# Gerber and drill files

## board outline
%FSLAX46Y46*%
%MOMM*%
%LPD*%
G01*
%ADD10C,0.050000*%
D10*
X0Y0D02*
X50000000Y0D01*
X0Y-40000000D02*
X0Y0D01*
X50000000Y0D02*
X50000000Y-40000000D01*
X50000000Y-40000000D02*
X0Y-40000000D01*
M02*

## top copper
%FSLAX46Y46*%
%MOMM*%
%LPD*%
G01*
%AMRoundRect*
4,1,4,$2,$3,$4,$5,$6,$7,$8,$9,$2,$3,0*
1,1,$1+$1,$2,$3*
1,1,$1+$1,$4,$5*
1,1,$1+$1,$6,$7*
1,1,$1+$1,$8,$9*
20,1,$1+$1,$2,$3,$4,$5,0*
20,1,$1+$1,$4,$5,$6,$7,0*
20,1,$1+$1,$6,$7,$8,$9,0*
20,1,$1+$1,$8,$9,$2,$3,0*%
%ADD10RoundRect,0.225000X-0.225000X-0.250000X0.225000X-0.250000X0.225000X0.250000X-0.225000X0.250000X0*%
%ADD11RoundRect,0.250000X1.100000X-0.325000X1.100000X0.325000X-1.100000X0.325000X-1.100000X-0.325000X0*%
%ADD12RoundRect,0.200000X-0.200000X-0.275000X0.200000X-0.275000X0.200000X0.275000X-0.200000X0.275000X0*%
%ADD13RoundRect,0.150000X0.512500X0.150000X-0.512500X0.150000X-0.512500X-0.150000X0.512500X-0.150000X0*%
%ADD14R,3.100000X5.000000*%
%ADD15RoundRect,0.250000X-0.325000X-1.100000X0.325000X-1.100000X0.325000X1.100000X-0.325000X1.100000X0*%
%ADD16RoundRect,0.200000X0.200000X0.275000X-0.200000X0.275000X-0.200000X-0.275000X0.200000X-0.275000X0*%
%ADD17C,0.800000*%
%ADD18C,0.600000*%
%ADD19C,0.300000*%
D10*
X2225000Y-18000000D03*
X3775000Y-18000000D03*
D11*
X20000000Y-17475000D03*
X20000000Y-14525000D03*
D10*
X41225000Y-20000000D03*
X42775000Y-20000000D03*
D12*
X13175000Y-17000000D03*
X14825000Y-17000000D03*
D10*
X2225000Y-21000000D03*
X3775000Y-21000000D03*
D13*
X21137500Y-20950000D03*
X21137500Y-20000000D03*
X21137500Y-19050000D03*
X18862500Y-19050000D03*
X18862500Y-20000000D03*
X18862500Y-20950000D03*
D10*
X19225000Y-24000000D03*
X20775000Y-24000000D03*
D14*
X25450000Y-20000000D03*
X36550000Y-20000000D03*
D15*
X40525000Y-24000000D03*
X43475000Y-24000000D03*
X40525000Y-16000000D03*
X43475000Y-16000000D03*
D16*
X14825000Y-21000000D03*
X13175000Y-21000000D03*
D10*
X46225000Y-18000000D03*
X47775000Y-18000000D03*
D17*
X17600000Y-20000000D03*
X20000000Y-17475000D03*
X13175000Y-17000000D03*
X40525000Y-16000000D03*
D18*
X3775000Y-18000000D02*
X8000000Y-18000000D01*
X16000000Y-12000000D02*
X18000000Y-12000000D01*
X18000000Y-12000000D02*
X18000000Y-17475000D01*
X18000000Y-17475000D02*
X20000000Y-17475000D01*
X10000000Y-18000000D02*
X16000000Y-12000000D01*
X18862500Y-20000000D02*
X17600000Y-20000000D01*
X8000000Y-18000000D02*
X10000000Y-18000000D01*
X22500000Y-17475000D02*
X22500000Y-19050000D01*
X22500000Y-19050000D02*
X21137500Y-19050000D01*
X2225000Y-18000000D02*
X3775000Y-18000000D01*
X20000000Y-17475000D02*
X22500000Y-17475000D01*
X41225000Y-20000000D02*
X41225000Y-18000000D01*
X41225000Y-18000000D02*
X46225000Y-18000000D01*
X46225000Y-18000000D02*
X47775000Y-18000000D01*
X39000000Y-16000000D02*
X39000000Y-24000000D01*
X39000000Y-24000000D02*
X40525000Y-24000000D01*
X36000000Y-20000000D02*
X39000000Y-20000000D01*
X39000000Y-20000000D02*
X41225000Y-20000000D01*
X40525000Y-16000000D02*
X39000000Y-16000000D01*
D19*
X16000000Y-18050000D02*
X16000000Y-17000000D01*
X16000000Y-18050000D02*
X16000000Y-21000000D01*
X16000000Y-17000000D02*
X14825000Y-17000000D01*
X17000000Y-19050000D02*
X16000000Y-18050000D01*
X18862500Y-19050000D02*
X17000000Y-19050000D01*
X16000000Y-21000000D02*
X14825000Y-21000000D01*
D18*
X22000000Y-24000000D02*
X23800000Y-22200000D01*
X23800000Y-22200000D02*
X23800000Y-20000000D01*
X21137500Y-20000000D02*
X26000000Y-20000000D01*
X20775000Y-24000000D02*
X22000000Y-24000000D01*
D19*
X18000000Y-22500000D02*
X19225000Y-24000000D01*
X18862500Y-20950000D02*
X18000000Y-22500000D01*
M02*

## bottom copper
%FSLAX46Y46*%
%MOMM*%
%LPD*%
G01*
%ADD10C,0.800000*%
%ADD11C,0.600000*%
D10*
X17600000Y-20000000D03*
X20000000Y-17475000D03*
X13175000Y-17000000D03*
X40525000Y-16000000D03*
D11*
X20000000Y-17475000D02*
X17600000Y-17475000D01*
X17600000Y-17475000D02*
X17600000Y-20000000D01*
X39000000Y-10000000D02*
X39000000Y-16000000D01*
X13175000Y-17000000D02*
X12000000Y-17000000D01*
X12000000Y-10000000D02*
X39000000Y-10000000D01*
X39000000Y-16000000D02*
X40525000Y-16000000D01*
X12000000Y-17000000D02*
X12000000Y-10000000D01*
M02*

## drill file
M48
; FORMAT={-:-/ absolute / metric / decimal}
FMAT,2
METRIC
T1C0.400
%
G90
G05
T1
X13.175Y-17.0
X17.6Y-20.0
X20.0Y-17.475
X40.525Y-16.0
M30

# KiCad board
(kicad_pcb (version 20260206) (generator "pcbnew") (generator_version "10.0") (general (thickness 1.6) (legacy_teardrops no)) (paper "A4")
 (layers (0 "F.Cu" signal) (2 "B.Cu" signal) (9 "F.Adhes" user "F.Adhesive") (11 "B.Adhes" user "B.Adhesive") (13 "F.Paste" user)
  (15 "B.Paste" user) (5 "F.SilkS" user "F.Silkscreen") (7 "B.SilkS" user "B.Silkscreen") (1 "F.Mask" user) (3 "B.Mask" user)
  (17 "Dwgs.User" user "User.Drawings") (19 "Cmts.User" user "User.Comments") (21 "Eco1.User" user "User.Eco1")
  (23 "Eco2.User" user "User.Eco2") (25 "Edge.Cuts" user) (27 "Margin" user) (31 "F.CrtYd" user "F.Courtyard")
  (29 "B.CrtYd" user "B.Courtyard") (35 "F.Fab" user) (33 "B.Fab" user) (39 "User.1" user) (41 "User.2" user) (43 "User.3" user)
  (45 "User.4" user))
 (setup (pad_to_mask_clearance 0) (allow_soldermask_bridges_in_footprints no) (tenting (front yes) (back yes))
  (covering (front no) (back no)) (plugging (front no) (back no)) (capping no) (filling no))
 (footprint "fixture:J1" (layer "F.Cu") (at 3 18)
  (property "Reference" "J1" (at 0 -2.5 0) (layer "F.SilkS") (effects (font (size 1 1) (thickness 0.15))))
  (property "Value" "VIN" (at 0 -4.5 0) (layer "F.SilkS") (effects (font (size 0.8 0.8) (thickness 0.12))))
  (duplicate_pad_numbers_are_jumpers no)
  (pad "1" smd roundrect (at -0.775 0) (size 0.9 0.95) (layers "F.Cu" "F.Mask" "F.Paste") (roundrect_rratio 0.25) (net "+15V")
   (thermal_bridge_angle 45))
  (pad "2" smd roundrect (at 0.775 0) (size 0.9 0.95) (layers "F.Cu" "F.Mask" "F.Paste") (roundrect_rratio 0.25) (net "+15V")
   (thermal_bridge_angle 45)))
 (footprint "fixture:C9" (layer "F.Cu") (at 20 16 90)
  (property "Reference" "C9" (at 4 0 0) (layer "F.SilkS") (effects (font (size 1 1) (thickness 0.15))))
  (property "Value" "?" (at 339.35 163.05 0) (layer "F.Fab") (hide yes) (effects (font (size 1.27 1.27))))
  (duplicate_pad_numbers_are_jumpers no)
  (pad "1" smd roundrect (at -1.475 0 90) (size 1.15 2.7) (layers "F.Cu" "F.Mask" "F.Paste") (roundrect_rratio 0.217391) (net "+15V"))
  (pad "2" smd roundrect (at 1.475 0 90) (size 1.15 2.7) (layers "F.Cu" "F.Mask" "F.Paste") (roundrect_rratio 0.217391) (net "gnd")))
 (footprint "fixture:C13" (layer "F.Cu") (at 42 20)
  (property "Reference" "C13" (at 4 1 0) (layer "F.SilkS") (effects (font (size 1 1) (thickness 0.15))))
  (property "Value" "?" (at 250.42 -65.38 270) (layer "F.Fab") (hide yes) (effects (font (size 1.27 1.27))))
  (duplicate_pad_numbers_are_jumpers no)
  (pad "1" smd roundrect (at -0.775 0) (size 0.9 0.95) (layers "F.Cu" "F.Mask" "F.Paste") (roundrect_rratio 0.25) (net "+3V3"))
  (pad "2" smd roundrect (at 0.775 0) (size 0.9 0.95) (layers "F.Cu" "F.Mask" "F.Paste") (roundrect_rratio 0.25) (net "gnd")))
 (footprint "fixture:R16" (layer "F.Cu") (at 14 17)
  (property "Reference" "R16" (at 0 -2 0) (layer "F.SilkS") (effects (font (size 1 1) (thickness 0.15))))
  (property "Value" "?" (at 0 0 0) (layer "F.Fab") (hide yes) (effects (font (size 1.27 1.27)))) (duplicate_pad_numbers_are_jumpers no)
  (pad "1" smd roundrect (at -0.825 0) (size 0.8 0.95) (layers "F.Cu" "F.Mask" "F.Paste") (roundrect_rratio 0.25) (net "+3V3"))
  (pad "2" smd roundrect (at 0.825 0) (size 0.8 0.95) (layers "F.Cu" "F.Mask" "F.Paste") (roundrect_rratio 0.25) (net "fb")))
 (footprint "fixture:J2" (layer "F.Cu") (at 3 21)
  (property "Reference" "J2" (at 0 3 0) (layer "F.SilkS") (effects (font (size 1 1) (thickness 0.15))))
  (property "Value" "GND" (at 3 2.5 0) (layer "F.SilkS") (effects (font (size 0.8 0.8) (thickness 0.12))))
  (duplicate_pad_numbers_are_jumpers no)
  (pad "1" smd roundrect (at -0.775 0) (size 0.9 0.95) (layers "F.Cu" "F.Mask" "F.Paste") (roundrect_rratio 0.25) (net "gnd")
   (thermal_bridge_angle 45))
  (pad "2" smd roundrect (at 0.775 0) (size 0.9 0.95) (layers "F.Cu" "F.Mask" "F.Paste") (roundrect_rratio 0.25) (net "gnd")
   (thermal_bridge_angle 45)))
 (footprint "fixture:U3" (layer "F.Cu") (at 20 20 180)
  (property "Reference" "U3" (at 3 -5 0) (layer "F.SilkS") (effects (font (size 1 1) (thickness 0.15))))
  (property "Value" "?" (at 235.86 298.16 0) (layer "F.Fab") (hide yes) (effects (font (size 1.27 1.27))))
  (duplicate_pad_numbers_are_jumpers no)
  (pad "1" smd roundrect (at -1.1375 -0.95 180) (size 1.325 0.6) (layers "F.Cu" "F.Mask" "F.Paste") (roundrect_rratio 0.25) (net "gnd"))
  (pad "2" smd roundrect (at -1.1375 0 180) (size 1.325 0.6) (layers "F.Cu" "F.Mask" "F.Paste") (roundrect_rratio 0.25) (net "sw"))
  (pad "3" smd roundrect (at -1.1375 0.95 180) (size 1.325 0.6) (layers "F.Cu" "F.Mask" "F.Paste") (roundrect_rratio 0.25) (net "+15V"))
  (pad "4" smd roundrect (at 1.1375 0.95 180) (size 1.325 0.6) (layers "F.Cu" "F.Mask" "F.Paste") (roundrect_rratio 0.25) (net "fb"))
  (pad "5" smd roundrect (at 1.1375 0 180) (size 1.325 0.6) (layers "F.Cu" "F.Mask" "F.Paste") (roundrect_rratio 0.25) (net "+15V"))
  (pad "6" smd roundrect (at 1.1375 -0.95 180) (size 1.325 0.6) (layers "F.Cu" "F.Mask" "F.Paste") (roundrect_rratio 0.25) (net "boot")))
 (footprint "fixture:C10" (layer "F.Cu") (at 20 24)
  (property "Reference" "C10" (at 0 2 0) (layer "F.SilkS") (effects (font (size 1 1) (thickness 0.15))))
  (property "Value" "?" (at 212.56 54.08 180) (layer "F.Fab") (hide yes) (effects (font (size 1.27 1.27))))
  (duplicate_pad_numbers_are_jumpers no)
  (pad "1" smd roundrect (at -0.775 0) (size 0.9 0.95) (layers "F.Cu" "F.Mask" "F.Paste") (roundrect_rratio 0.25) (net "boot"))
  (pad "2" smd roundrect (at 0.775 0) (size 0.9 0.95) (layers "F.Cu" "F.Mask" "F.Paste") (roundrect_rratio 0.25) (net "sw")))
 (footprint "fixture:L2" (layer "F.Cu") (at 31 20)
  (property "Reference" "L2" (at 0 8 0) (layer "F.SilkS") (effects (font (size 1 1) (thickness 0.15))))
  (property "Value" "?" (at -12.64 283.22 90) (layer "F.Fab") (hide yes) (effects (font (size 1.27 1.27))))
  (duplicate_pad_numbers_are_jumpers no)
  (pad "1" smd rect (at -5.55 0) (size 3.1 5) (layers "F.Cu" "F.Mask" "F.Paste") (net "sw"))
  (pad "2" smd rect (at 5.55 0) (size 3.1 5) (layers "F.Cu" "F.Mask" "F.Paste") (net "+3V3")))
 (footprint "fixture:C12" (layer "F.Cu") (at 42 24)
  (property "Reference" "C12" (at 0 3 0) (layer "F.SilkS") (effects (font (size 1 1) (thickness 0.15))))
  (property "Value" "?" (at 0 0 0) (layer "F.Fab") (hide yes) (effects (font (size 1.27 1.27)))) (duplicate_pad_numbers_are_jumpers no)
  (pad "1" smd roundrect (at -1.475 0) (size 1.15 2.7) (layers "F.Cu" "F.Mask" "F.Paste") (roundrect_rratio 0.217391) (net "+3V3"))
  (pad "2" smd roundrect (at 1.475 0) (size 1.15 2.7) (layers "F.Cu" "F.Mask" "F.Paste") (roundrect_rratio 0.217391) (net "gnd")))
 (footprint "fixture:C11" (layer "F.Cu") (at 42 16)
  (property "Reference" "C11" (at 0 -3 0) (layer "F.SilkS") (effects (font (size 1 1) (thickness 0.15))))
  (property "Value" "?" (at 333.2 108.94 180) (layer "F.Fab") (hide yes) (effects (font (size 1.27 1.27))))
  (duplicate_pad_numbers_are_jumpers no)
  (pad "1" smd roundrect (at -1.475 0) (size 1.15 2.7) (layers "F.Cu" "F.Mask" "F.Paste") (roundrect_rratio 0.217391) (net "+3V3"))
  (pad "2" smd roundrect (at 1.475 0) (size 1.15 2.7) (layers "F.Cu" "F.Mask" "F.Paste") (roundrect_rratio 0.217391) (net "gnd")))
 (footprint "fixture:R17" (layer "F.Cu") (at 14 21 180)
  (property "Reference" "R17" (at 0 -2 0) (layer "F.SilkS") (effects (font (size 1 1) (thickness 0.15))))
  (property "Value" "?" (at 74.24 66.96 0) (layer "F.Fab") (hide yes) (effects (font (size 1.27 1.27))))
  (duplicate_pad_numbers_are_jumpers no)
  (pad "1" smd roundrect (at -0.825 0 180) (size 0.8 0.95) (layers "F.Cu" "F.Mask" "F.Paste") (roundrect_rratio 0.25) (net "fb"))
  (pad "2" smd roundrect (at 0.825 0 180) (size 0.8 0.95) (layers "F.Cu" "F.Mask" "F.Paste") (roundrect_rratio 0.25) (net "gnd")))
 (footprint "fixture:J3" (layer "F.Cu") (at 47 18)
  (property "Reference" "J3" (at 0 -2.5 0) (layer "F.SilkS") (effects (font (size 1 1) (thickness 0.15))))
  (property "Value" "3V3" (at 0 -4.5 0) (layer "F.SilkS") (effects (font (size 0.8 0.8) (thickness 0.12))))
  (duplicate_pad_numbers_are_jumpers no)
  (pad "1" smd roundrect (at -0.775 0) (size 0.9 0.95) (layers "F.Cu" "F.Mask" "F.Paste") (roundrect_rratio 0.25) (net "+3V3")
   (thermal_bridge_angle 45))
  (pad "2" smd roundrect (at 0.775 0) (size 0.9 0.95) (layers "F.Cu" "F.Mask" "F.Paste") (roundrect_rratio 0.25) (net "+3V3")
   (thermal_bridge_angle 45)))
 (gr_line (start 0 0) (end 50 0) (stroke (width 0.05) (type default)) (layer "Edge.Cuts"))
 (gr_line (start 0 40) (end 0 0) (stroke (width 0.05) (type default)) (layer "Edge.Cuts"))
 (gr_line (start 50 0) (end 50 40) (stroke (width 0.05) (type default)) (layer "Edge.Cuts"))
 (gr_line (start 50 40) (end 0 40) (stroke (width 0.05) (type default)) (layer "Edge.Cuts"))
 (segment (start 3.775 18) (end 8 18) (width 0.6) (layer "F.Cu") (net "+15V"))
 (segment (start 16 12) (end 18 12) (width 0.6) (layer "F.Cu") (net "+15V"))
 (segment (start 18 12) (end 18 17.475) (width 0.6) (layer "F.Cu") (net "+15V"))
 (segment (start 18 17.475) (end 20 17.475) (width 0.6) (layer "F.Cu") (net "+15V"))
 (segment (start 10 18) (end 16 12) (width 0.6) (layer "F.Cu") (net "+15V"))
 (segment (start 18.8625 20) (end 17.6 20) (width 0.6) (layer "F.Cu") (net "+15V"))
 (segment (start 8 18) (end 10 18) (width 0.6) (layer "F.Cu") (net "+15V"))
 (segment (start 22.5 17.475) (end 22.5 19.05) (width 0.6) (layer "F.Cu") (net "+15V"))
 (segment (start 22.5 19.05) (end 21.1375 19.05) (width 0.6) (layer "F.Cu") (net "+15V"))
 (segment (start 2.225 18) (end 3.775 18) (width 0.6) (layer "F.Cu") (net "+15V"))
 (segment (start 20 17.475) (end 22.5 17.475) (width 0.6) (layer "F.Cu") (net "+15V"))
 (via (at 17.6 20) (size 0.8) (drill 0.4) (layers "F.Cu" "B.Cu") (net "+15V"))
 (via (at 20 17.475) (size 0.8) (drill 0.4) (layers "F.Cu" "B.Cu") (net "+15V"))
 (segment (start 20 17.475) (end 17.6 17.475) (width 0.6) (layer "B.Cu") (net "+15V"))
 (segment (start 17.6 17.475) (end 17.6 20) (width 0.6) (layer "B.Cu") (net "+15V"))
 (segment (start 41.225 20) (end 41.225 18) (width 0.6) (layer "F.Cu") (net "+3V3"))
 (segment (start 41.225 18) (end 46.225 18) (width 0.6) (layer "F.Cu") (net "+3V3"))
 (segment (start 46.225 18) (end 47.775 18) (width 0.6) (layer "F.Cu") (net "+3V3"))
 (segment (start 39 16) (end 39 24) (width 0.6) (layer "F.Cu") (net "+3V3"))
 (segment (start 39 24) (end 40.525 24) (width 0.6) (layer "F.Cu") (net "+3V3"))
 (segment (start 36 20) (end 39 20) (width 0.6) (layer "F.Cu") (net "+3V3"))
 (segment (start 39 20) (end 41.225 20) (width 0.6) (layer "F.Cu") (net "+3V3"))
 (segment (start 40.525 16) (end 39 16) (width 0.6) (layer "F.Cu") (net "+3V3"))
 (via (at 13.175 17) (size 0.8) (drill 0.4) (layers "F.Cu" "B.Cu") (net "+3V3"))
 (via (at 40.525 16) (size 0.8) (drill 0.4) (layers "F.Cu" "B.Cu") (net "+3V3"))
 (segment (start 39 10) (end 39 16) (width 0.6) (layer "B.Cu") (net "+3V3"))
 (segment (start 13.175 17) (end 12 17) (width 0.6) (layer "B.Cu") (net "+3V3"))
 (segment (start 12 10) (end 39 10) (width 0.6) (layer "B.Cu") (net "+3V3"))
 (segment (start 39 16) (end 40.525 16) (width 0.6) (layer "B.Cu") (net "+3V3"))
 (segment (start 12 17) (end 12 10) (width 0.6) (layer "B.Cu") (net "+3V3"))
 (segment (start 16 18.05) (end 16 17) (width 0.3) (layer "F.Cu") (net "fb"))
 (segment (start 16 18.05) (end 16 21) (width 0.3) (layer "F.Cu") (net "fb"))
 (segment (start 16 17) (end 14.825 17) (width 0.3) (layer "F.Cu") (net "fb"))
 (segment (start 17 19.05) (end 16 18.05) (width 0.3) (layer "F.Cu") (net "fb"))
 (segment (start 18.8625 19.05) (end 17 19.05) (width 0.3) (layer "F.Cu") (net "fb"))
 (segment (start 16 21) (end 14.825 21) (width 0.3) (layer "F.Cu") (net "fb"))
 (segment (start 22 24) (end 23.8 22.2) (width 0.6) (layer "F.Cu") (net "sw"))
 (segment (start 23.8 22.2) (end 23.8 20) (width 0.6) (layer "F.Cu") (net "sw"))
 (segment (start 21.1375 20) (end 26 20) (width 0.6) (layer "F.Cu") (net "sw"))
 (segment (start 20.775 24) (end 22 24) (width 0.6) (layer "F.Cu") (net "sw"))
 (segment (start 18 22.5) (end 19.225 24) (width 0.3) (layer "F.Cu") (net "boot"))
 (segment (start 18.8625 20.95) (end 18 22.5) (width 0.3) (layer "F.Cu") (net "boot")))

